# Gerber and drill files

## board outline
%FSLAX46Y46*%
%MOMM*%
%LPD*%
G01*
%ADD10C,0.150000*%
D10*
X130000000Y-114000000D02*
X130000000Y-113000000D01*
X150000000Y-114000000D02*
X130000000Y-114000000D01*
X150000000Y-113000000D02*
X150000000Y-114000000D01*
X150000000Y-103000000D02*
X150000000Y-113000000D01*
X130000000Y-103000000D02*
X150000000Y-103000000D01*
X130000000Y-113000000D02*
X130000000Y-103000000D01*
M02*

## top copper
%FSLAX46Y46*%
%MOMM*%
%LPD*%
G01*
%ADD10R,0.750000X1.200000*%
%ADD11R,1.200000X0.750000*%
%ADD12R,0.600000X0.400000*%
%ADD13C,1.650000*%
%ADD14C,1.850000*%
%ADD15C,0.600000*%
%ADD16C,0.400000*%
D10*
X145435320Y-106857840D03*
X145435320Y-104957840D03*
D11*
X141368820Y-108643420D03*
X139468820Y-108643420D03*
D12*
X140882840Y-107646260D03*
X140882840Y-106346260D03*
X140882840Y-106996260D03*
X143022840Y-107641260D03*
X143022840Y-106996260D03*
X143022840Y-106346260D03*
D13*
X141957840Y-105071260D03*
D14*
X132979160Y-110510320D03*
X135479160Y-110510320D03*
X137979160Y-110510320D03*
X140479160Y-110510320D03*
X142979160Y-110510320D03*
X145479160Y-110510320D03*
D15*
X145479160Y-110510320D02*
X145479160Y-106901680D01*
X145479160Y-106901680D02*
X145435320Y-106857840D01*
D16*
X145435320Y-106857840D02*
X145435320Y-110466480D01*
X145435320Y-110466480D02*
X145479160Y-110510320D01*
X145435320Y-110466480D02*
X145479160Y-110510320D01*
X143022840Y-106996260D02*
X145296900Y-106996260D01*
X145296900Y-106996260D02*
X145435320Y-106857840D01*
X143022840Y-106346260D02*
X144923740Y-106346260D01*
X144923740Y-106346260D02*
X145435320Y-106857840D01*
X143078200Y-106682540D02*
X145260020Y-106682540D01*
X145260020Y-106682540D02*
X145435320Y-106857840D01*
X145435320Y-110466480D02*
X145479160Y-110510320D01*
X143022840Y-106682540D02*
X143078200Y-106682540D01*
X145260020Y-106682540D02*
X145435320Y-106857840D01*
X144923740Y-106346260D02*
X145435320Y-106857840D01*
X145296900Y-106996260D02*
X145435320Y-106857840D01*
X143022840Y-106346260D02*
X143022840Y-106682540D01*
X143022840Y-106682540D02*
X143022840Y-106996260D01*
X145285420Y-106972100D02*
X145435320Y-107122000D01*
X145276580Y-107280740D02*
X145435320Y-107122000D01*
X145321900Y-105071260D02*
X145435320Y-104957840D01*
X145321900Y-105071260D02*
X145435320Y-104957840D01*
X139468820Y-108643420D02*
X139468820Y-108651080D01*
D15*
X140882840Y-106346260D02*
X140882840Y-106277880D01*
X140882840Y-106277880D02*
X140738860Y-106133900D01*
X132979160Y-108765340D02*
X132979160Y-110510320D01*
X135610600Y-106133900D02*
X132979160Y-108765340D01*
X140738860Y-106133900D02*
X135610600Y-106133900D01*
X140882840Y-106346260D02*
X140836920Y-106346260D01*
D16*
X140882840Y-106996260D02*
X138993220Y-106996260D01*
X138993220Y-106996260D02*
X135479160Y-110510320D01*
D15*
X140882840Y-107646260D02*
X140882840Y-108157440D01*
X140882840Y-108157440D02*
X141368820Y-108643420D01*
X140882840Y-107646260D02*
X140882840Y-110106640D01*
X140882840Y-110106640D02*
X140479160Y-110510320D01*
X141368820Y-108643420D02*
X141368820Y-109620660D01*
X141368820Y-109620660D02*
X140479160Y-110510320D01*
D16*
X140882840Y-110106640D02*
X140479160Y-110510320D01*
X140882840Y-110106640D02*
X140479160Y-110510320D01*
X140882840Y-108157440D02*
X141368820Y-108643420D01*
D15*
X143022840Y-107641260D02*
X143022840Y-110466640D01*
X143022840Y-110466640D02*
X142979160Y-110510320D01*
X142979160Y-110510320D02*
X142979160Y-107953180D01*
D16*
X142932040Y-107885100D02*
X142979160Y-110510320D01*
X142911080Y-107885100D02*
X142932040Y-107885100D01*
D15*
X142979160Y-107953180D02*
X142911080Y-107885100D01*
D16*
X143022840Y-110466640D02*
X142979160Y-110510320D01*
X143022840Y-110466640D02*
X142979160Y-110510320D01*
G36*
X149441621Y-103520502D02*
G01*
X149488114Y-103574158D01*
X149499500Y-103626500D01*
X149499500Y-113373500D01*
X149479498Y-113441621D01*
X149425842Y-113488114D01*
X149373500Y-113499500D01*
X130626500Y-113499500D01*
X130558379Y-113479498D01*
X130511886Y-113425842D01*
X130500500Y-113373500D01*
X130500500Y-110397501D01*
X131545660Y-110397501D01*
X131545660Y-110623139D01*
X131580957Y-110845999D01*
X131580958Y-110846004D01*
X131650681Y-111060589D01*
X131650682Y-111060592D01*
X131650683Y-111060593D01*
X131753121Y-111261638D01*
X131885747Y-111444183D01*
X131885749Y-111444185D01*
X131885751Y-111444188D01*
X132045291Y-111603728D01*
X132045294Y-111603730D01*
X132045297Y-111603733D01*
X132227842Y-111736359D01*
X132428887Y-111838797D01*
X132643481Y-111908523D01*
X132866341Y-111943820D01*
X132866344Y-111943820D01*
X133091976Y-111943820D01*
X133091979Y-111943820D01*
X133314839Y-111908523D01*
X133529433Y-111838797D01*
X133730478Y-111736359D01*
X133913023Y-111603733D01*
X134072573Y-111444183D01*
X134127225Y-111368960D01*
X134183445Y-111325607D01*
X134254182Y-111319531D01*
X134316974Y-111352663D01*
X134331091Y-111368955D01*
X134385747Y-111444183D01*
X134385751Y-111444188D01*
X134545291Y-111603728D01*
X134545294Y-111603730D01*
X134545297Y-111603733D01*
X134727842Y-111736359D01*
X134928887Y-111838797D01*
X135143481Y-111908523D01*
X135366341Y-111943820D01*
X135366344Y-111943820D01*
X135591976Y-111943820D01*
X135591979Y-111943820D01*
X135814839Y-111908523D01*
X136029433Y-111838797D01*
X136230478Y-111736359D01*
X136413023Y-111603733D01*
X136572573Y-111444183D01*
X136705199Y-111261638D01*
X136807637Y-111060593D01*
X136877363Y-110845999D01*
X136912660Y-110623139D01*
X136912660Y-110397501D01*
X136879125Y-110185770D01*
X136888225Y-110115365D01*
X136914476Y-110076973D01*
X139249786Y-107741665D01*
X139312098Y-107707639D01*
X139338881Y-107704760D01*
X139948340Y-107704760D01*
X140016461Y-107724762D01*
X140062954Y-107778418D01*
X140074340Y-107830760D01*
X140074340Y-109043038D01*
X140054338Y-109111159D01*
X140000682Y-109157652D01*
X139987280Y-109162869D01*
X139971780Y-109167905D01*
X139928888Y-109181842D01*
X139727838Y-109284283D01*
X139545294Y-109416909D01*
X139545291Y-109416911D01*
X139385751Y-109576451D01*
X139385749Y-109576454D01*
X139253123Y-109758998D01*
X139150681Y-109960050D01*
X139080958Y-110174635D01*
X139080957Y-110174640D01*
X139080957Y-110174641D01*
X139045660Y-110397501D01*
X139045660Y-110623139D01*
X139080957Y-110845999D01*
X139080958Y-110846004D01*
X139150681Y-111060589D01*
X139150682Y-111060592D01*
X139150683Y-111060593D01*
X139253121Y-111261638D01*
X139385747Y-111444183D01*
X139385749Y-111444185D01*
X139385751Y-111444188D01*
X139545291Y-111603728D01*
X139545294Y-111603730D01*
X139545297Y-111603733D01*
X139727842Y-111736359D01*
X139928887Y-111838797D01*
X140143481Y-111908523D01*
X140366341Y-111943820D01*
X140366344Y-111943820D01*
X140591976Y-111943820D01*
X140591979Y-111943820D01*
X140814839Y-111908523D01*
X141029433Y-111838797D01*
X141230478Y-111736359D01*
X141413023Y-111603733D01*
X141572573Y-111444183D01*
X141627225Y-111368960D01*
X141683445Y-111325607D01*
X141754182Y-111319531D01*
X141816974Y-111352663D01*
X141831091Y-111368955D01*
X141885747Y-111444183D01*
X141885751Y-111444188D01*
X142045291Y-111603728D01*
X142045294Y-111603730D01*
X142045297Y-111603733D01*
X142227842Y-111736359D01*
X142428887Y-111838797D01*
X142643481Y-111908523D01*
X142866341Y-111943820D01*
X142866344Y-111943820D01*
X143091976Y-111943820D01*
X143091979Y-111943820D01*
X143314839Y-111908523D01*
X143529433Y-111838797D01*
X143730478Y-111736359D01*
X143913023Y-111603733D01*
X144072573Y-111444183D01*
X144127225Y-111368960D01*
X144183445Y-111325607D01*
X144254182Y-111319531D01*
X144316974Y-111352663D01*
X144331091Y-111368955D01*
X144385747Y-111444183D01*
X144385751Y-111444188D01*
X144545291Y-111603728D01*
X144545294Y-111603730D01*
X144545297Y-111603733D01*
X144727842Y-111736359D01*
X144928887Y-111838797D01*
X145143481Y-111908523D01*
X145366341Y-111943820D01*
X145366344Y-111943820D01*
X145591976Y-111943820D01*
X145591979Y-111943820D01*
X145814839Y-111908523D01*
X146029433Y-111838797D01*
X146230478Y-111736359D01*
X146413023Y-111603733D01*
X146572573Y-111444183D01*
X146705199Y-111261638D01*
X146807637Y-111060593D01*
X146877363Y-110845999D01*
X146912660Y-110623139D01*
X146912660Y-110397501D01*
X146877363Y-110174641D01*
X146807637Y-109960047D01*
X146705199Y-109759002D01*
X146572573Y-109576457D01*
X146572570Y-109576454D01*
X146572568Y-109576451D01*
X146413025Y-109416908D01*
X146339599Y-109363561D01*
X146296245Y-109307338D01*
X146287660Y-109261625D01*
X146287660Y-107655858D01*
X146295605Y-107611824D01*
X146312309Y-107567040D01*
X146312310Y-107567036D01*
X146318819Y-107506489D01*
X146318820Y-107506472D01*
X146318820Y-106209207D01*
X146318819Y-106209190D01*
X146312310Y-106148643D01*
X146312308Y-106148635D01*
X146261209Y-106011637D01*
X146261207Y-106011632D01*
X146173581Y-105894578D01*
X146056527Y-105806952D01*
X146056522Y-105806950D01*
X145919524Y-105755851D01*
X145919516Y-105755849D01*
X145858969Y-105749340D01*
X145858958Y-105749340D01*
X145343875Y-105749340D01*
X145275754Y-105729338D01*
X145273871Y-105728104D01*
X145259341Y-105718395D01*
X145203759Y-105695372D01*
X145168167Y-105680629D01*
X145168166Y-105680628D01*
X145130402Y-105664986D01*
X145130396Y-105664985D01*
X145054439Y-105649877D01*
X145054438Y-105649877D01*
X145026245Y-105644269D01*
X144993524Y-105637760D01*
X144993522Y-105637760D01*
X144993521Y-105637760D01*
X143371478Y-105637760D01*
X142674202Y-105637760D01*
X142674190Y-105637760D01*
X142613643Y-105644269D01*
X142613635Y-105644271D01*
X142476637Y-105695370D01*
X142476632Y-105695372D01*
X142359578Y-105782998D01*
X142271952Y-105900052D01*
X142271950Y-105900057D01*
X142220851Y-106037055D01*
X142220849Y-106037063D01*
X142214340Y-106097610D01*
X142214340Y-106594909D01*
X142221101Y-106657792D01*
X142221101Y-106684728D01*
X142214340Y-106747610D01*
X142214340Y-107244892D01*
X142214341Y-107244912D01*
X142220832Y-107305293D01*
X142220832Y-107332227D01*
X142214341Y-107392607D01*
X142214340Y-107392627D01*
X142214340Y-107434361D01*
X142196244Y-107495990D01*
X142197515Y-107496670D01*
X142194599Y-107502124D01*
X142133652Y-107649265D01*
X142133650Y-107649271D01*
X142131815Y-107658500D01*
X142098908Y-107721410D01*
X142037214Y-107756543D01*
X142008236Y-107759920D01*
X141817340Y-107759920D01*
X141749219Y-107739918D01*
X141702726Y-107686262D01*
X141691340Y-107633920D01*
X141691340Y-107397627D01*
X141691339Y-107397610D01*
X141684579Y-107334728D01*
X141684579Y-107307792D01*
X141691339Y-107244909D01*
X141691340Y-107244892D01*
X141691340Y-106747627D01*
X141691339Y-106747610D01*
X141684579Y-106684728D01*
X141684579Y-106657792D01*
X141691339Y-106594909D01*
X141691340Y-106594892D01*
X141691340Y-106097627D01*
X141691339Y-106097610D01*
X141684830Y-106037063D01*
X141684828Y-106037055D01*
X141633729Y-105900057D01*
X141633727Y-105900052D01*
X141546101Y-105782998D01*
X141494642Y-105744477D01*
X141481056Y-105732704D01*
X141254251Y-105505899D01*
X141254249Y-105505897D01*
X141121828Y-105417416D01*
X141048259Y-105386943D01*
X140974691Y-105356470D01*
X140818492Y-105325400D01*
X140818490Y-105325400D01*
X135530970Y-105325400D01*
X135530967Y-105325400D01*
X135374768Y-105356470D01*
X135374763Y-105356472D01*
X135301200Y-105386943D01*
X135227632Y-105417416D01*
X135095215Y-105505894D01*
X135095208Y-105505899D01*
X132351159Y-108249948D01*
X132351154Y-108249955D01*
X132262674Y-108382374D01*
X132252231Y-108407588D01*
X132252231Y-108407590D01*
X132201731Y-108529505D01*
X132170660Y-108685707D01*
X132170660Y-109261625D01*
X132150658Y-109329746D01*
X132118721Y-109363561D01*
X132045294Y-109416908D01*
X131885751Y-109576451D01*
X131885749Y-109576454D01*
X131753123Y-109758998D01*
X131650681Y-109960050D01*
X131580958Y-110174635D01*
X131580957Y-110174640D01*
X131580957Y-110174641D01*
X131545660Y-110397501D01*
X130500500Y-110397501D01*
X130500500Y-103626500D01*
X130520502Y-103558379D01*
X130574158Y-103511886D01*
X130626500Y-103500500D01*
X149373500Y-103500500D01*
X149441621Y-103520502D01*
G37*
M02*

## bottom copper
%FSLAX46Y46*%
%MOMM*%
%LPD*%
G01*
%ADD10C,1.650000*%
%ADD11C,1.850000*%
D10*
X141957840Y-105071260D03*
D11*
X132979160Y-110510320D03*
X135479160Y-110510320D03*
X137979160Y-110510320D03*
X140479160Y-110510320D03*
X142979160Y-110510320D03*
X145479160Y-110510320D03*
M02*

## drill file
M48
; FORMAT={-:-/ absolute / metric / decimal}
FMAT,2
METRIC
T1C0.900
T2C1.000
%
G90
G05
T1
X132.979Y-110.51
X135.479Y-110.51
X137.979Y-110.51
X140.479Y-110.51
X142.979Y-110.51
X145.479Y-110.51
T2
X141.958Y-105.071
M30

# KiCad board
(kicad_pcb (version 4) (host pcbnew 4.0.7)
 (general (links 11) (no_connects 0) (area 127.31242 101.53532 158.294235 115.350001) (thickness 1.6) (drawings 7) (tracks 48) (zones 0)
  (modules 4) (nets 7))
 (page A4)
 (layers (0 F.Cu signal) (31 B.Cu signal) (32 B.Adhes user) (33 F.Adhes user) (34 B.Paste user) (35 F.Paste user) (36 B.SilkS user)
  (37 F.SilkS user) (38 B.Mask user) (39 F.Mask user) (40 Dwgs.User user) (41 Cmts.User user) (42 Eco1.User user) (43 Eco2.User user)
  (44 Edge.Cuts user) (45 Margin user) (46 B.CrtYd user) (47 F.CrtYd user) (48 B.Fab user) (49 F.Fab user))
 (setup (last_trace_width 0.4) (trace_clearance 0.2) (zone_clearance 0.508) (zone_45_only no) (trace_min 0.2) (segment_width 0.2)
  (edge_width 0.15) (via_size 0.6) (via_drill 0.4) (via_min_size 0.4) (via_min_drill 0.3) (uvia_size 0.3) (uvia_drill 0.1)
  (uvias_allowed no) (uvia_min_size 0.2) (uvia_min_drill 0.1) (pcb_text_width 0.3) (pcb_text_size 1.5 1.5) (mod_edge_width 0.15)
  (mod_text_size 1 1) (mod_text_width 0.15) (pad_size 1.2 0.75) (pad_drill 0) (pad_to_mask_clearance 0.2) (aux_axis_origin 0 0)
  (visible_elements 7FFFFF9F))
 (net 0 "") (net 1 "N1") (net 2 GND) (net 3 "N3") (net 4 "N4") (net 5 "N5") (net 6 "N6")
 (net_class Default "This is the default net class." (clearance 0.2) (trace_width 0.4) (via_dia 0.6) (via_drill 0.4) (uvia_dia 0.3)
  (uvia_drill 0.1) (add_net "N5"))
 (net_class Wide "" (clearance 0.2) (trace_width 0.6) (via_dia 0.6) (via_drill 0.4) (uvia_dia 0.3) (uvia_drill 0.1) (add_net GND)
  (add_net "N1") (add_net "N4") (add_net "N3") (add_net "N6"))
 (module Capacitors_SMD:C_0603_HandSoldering (layer F.Cu) (at 145.43532 105.90784 90)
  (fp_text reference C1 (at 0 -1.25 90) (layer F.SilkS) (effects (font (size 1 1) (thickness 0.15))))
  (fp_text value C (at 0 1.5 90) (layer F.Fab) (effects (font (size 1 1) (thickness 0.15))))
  (pad 1 smd rect (at -0.95 0 90) (size 1.2 0.75) (layers F.Cu F.Paste F.Mask) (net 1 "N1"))
  (pad 2 smd rect (at 0.95 0 90) (size 1.2 0.75) (layers F.Cu F.Paste F.Mask) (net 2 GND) (zone_connect 2)))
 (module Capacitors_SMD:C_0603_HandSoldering (layer F.Cu) (at 140.41882 108.64342 180)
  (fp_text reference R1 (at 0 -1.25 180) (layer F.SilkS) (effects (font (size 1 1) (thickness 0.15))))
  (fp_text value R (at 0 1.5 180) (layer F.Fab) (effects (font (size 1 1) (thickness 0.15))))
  (pad 1 smd rect (at -0.95 0 180) (size 1.2 0.75) (layers F.Cu F.Paste F.Mask) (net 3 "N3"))
  (pad 2 smd rect (at 0.95 0 180) (size 1.2 0.75) (layers F.Cu F.Paste F.Mask) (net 2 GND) (zone_connect 2)))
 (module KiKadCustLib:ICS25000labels (layer F.Cu) (at 148.45284 105.96626)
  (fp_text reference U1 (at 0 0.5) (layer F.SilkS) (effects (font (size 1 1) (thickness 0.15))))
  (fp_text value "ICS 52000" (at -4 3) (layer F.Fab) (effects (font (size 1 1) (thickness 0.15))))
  (pad 7 smd rect (at -7.57 1.68) (size 0.6 0.4) (layers F.Cu F.Paste F.Mask) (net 3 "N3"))
  (pad 5 smd rect (at -7.57 0.38) (size 0.6 0.4) (layers F.Cu F.Paste F.Mask) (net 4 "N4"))
  (pad 6 smd rect (at -7.57 1.03) (size 0.6 0.4) (layers F.Cu F.Paste F.Mask) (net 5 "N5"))
  (pad 1 smd rect (at -5.43 1.675) (size 0.6 0.4) (layers F.Cu F.Paste F.Mask) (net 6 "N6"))
  (pad 2 smd rect (at -5.43 1.03) (size 0.6 0.4) (layers F.Cu F.Paste F.Mask) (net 1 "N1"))
  (pad 3 smd rect (at -5.43 0.38) (size 0.6 0.4) (layers F.Cu F.Paste F.Mask) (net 1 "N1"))
  (pad 4 thru_hole circle (at -6.495 -0.895) (size 1.65 1.65) (drill 1) (layers *.Cu *.Mask) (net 2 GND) (zone_connect 2)))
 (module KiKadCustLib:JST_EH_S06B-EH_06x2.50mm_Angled (layer F.Cu) (at 132.97916 110.51032)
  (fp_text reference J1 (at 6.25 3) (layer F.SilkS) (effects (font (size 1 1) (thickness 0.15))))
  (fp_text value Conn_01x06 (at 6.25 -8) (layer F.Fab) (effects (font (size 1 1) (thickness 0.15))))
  (pad 2 thru_hole circle (at 0 0) (size 1.85 1.85) (drill 0.9) (layers *.Cu *.Mask) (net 4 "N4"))
  (pad 3 thru_hole circle (at 2.5 0) (size 1.85 1.85) (drill 0.9) (layers *.Cu *.Mask) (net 5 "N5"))
  (pad 6 thru_hole circle (at 5 0) (size 1.85 1.85) (drill 0.9) (layers *.Cu *.Mask) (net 2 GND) (zone_connect 2))
  (pad 4 thru_hole circle (at 7.5 0) (size 1.85 1.85) (drill 0.9) (layers *.Cu *.Mask) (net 3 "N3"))
  (pad 5 thru_hole circle (at 10 0) (size 1.85 1.85) (drill 0.9) (layers *.Cu *.Mask) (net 6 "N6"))
  (pad 1 thru_hole circle (at 12.5 0) (size 1.85 1.85) (drill 0.9) (layers *.Cu *.Mask) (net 1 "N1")))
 (gr_line (start 130 114) (end 130 113) (angle 90) (layer Edge.Cuts) (width 0.15))
 (gr_line (start 150 114) (end 130 114) (angle 90) (layer Edge.Cuts) (width 0.15))
 (gr_line (start 150 113) (end 150 114) (angle 90) (layer Edge.Cuts) (width 0.15))
 (gr_line (start 150 103) (end 150 113) (angle 90) (layer Edge.Cuts) (width 0.15))
 (gr_line (start 130 103) (end 150 103) (angle 90) (layer Edge.Cuts) (width 0.15))
 (gr_line (start 130 113) (end 130 103) (angle 90) (layer Edge.Cuts) (width 0.15))
 (segment (start 145.47916 110.51032) (end 145.47916 106.90168) (width 0.6) (layer F.Cu) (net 1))
 (segment (start 145.47916 106.90168) (end 145.43532 106.85784) (width 0.6) (layer F.Cu) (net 1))
 (segment (start 145.43532 106.85784) (end 145.43532 110.46648) (width 0.4) (layer F.Cu) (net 1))
 (segment (start 145.43532 110.46648) (end 145.47916 110.51032) (width 0.4) (layer F.Cu) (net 1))
 (segment (start 145.43532 110.46648) (end 145.47916 110.51032) (width 0.4) (layer F.Cu) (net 1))
 (segment (start 143.02284 106.99626) (end 145.2969 106.99626) (width 0.4) (layer F.Cu) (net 1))
 (segment (start 145.2969 106.99626) (end 145.43532 106.85784) (width 0.4) (layer F.Cu) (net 1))
 (segment (start 143.02284 106.34626) (end 144.92374 106.34626) (width 0.4) (layer F.Cu) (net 1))
 (segment (start 144.92374 106.34626) (end 145.43532 106.85784) (width 0.4) (layer F.Cu) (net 1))
 (segment (start 143.0782 106.68254) (end 145.26002 106.68254) (width 0.4) (layer F.Cu) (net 1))
 (segment (start 145.26002 106.68254) (end 145.43532 106.85784) (width 0.4) (layer F.Cu) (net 1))
 (segment (start 145.43532 110.46648) (end 145.47916 110.51032) (width 0.4) (layer F.Cu) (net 1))
 (segment (start 143.02284 106.68254) (end 143.0782 106.68254) (width 0.4) (layer F.Cu) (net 1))
 (segment (start 145.26002 106.68254) (end 145.43532 106.85784) (width 0.4) (layer F.Cu) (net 1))
 (segment (start 144.92374 106.34626) (end 145.43532 106.85784) (width 0.4) (layer F.Cu) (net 1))
 (segment (start 145.2969 106.99626) (end 145.43532 106.85784) (width 0.4) (layer F.Cu) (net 1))
 (segment (start 143.02284 106.34626) (end 143.02284 106.68254) (width 0.4) (layer F.Cu) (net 1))
 (segment (start 143.02284 106.68254) (end 143.02284 106.99626) (width 0.4) (layer F.Cu) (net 1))
 (segment (start 145.28542 106.9721) (end 145.43532 107.122) (width 0.4) (layer F.Cu) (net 1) (status 30))
 (segment (start 145.27658 107.28074) (end 145.43532 107.122) (width 0.4) (layer F.Cu) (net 1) (status 30))
 (segment (start 145.3219 105.07126) (end 145.43532 104.95784) (width 0.4) (layer F.Cu) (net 2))
 (segment (start 145.3219 105.07126) (end 145.43532 104.95784) (width 0.4) (layer F.Cu) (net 2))
 (segment (start 139.46882 108.64342) (end 139.46882 108.65108) (width 0.4) (layer F.Cu) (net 2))
 (segment (start 140.88284 106.34626) (end 140.88284 106.27788) (width 0.6) (layer F.Cu) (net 4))
 (segment (start 140.88284 106.27788) (end 140.73886 106.1339) (width 0.6) (layer F.Cu) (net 4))
 (segment (start 132.97916 108.76534) (end 132.97916 110.51032) (width 0.6) (layer F.Cu) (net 4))
 (segment (start 135.6106 106.1339) (end 132.97916 108.76534) (width 0.6) (layer F.Cu) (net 4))
 (segment (start 140.73886 106.1339) (end 135.6106 106.1339) (width 0.6) (layer F.Cu) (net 4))
 (segment (start 140.88284 106.34626) (end 140.83692 106.34626) (width 0.6) (layer F.Cu) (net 4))
 (segment (start 140.88284 106.99626) (end 138.99322 106.99626) (width 0.4) (layer F.Cu) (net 5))
 (segment (start 138.99322 106.99626) (end 135.47916 110.51032) (width 0.4) (layer F.Cu) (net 5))
 (segment (start 140.88284 107.64626) (end 140.88284 108.15744) (width 0.6) (layer F.Cu) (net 3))
 (segment (start 140.88284 108.15744) (end 141.36882 108.64342) (width 0.6) (layer F.Cu) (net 3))
 (segment (start 140.88284 107.64626) (end 140.88284 110.10664) (width 0.6) (layer F.Cu) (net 3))
 (segment (start 140.88284 110.10664) (end 140.47916 110.51032) (width 0.6) (layer F.Cu) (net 3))
 (segment (start 141.36882 108.64342) (end 141.36882 109.62066) (width 0.6) (layer F.Cu) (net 3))
 (segment (start 141.36882 109.62066) (end 140.47916 110.51032) (width 0.6) (layer F.Cu) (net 3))
 (segment (start 140.88284 110.10664) (end 140.47916 110.51032) (width 0.4) (layer F.Cu) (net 3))
 (segment (start 140.88284 110.10664) (end 140.47916 110.51032) (width 0.4) (layer F.Cu) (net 3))
 (segment (start 140.88284 108.15744) (end 141.36882 108.64342) (width 0.4) (layer F.Cu) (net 3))
 (segment (start 143.02284 107.64126) (end 143.02284 110.46664) (width 0.6) (layer F.Cu) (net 6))
 (segment (start 143.02284 110.46664) (end 142.97916 110.51032) (width 0.6) (layer F.Cu) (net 6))
 (segment (start 142.97916 110.51032) (end 142.97916 107.95318) (width 0.6) (layer F.Cu) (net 6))
 (segment (start 142.93204 107.8851) (end 142.97916 110.51032) (width 0.4) (layer F.Cu) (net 6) (status 10))
 (segment (start 142.91108 107.8851) (end 142.93204 107.8851) (width 0.4) (layer F.Cu) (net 6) (status 30))
 (segment (start 142.97916 107.95318) (end 142.91108 107.8851) (width 0.6) (layer F.Cu) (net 6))
 (segment (start 143.02284 110.46664) (end 142.97916 110.51032) (width 0.4) (layer F.Cu) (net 6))
 (segment (start 143.02284 110.46664) (end 142.97916 110.51032) (width 0.4) (layer F.Cu) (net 6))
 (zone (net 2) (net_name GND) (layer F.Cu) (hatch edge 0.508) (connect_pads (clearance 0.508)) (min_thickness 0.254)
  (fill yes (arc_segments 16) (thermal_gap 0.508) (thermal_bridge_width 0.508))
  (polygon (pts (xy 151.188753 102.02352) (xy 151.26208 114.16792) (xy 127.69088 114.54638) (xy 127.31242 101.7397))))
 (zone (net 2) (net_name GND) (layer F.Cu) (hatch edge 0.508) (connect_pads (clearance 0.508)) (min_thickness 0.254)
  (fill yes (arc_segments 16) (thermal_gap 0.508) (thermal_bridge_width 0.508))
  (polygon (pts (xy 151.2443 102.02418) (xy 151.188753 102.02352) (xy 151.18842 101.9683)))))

